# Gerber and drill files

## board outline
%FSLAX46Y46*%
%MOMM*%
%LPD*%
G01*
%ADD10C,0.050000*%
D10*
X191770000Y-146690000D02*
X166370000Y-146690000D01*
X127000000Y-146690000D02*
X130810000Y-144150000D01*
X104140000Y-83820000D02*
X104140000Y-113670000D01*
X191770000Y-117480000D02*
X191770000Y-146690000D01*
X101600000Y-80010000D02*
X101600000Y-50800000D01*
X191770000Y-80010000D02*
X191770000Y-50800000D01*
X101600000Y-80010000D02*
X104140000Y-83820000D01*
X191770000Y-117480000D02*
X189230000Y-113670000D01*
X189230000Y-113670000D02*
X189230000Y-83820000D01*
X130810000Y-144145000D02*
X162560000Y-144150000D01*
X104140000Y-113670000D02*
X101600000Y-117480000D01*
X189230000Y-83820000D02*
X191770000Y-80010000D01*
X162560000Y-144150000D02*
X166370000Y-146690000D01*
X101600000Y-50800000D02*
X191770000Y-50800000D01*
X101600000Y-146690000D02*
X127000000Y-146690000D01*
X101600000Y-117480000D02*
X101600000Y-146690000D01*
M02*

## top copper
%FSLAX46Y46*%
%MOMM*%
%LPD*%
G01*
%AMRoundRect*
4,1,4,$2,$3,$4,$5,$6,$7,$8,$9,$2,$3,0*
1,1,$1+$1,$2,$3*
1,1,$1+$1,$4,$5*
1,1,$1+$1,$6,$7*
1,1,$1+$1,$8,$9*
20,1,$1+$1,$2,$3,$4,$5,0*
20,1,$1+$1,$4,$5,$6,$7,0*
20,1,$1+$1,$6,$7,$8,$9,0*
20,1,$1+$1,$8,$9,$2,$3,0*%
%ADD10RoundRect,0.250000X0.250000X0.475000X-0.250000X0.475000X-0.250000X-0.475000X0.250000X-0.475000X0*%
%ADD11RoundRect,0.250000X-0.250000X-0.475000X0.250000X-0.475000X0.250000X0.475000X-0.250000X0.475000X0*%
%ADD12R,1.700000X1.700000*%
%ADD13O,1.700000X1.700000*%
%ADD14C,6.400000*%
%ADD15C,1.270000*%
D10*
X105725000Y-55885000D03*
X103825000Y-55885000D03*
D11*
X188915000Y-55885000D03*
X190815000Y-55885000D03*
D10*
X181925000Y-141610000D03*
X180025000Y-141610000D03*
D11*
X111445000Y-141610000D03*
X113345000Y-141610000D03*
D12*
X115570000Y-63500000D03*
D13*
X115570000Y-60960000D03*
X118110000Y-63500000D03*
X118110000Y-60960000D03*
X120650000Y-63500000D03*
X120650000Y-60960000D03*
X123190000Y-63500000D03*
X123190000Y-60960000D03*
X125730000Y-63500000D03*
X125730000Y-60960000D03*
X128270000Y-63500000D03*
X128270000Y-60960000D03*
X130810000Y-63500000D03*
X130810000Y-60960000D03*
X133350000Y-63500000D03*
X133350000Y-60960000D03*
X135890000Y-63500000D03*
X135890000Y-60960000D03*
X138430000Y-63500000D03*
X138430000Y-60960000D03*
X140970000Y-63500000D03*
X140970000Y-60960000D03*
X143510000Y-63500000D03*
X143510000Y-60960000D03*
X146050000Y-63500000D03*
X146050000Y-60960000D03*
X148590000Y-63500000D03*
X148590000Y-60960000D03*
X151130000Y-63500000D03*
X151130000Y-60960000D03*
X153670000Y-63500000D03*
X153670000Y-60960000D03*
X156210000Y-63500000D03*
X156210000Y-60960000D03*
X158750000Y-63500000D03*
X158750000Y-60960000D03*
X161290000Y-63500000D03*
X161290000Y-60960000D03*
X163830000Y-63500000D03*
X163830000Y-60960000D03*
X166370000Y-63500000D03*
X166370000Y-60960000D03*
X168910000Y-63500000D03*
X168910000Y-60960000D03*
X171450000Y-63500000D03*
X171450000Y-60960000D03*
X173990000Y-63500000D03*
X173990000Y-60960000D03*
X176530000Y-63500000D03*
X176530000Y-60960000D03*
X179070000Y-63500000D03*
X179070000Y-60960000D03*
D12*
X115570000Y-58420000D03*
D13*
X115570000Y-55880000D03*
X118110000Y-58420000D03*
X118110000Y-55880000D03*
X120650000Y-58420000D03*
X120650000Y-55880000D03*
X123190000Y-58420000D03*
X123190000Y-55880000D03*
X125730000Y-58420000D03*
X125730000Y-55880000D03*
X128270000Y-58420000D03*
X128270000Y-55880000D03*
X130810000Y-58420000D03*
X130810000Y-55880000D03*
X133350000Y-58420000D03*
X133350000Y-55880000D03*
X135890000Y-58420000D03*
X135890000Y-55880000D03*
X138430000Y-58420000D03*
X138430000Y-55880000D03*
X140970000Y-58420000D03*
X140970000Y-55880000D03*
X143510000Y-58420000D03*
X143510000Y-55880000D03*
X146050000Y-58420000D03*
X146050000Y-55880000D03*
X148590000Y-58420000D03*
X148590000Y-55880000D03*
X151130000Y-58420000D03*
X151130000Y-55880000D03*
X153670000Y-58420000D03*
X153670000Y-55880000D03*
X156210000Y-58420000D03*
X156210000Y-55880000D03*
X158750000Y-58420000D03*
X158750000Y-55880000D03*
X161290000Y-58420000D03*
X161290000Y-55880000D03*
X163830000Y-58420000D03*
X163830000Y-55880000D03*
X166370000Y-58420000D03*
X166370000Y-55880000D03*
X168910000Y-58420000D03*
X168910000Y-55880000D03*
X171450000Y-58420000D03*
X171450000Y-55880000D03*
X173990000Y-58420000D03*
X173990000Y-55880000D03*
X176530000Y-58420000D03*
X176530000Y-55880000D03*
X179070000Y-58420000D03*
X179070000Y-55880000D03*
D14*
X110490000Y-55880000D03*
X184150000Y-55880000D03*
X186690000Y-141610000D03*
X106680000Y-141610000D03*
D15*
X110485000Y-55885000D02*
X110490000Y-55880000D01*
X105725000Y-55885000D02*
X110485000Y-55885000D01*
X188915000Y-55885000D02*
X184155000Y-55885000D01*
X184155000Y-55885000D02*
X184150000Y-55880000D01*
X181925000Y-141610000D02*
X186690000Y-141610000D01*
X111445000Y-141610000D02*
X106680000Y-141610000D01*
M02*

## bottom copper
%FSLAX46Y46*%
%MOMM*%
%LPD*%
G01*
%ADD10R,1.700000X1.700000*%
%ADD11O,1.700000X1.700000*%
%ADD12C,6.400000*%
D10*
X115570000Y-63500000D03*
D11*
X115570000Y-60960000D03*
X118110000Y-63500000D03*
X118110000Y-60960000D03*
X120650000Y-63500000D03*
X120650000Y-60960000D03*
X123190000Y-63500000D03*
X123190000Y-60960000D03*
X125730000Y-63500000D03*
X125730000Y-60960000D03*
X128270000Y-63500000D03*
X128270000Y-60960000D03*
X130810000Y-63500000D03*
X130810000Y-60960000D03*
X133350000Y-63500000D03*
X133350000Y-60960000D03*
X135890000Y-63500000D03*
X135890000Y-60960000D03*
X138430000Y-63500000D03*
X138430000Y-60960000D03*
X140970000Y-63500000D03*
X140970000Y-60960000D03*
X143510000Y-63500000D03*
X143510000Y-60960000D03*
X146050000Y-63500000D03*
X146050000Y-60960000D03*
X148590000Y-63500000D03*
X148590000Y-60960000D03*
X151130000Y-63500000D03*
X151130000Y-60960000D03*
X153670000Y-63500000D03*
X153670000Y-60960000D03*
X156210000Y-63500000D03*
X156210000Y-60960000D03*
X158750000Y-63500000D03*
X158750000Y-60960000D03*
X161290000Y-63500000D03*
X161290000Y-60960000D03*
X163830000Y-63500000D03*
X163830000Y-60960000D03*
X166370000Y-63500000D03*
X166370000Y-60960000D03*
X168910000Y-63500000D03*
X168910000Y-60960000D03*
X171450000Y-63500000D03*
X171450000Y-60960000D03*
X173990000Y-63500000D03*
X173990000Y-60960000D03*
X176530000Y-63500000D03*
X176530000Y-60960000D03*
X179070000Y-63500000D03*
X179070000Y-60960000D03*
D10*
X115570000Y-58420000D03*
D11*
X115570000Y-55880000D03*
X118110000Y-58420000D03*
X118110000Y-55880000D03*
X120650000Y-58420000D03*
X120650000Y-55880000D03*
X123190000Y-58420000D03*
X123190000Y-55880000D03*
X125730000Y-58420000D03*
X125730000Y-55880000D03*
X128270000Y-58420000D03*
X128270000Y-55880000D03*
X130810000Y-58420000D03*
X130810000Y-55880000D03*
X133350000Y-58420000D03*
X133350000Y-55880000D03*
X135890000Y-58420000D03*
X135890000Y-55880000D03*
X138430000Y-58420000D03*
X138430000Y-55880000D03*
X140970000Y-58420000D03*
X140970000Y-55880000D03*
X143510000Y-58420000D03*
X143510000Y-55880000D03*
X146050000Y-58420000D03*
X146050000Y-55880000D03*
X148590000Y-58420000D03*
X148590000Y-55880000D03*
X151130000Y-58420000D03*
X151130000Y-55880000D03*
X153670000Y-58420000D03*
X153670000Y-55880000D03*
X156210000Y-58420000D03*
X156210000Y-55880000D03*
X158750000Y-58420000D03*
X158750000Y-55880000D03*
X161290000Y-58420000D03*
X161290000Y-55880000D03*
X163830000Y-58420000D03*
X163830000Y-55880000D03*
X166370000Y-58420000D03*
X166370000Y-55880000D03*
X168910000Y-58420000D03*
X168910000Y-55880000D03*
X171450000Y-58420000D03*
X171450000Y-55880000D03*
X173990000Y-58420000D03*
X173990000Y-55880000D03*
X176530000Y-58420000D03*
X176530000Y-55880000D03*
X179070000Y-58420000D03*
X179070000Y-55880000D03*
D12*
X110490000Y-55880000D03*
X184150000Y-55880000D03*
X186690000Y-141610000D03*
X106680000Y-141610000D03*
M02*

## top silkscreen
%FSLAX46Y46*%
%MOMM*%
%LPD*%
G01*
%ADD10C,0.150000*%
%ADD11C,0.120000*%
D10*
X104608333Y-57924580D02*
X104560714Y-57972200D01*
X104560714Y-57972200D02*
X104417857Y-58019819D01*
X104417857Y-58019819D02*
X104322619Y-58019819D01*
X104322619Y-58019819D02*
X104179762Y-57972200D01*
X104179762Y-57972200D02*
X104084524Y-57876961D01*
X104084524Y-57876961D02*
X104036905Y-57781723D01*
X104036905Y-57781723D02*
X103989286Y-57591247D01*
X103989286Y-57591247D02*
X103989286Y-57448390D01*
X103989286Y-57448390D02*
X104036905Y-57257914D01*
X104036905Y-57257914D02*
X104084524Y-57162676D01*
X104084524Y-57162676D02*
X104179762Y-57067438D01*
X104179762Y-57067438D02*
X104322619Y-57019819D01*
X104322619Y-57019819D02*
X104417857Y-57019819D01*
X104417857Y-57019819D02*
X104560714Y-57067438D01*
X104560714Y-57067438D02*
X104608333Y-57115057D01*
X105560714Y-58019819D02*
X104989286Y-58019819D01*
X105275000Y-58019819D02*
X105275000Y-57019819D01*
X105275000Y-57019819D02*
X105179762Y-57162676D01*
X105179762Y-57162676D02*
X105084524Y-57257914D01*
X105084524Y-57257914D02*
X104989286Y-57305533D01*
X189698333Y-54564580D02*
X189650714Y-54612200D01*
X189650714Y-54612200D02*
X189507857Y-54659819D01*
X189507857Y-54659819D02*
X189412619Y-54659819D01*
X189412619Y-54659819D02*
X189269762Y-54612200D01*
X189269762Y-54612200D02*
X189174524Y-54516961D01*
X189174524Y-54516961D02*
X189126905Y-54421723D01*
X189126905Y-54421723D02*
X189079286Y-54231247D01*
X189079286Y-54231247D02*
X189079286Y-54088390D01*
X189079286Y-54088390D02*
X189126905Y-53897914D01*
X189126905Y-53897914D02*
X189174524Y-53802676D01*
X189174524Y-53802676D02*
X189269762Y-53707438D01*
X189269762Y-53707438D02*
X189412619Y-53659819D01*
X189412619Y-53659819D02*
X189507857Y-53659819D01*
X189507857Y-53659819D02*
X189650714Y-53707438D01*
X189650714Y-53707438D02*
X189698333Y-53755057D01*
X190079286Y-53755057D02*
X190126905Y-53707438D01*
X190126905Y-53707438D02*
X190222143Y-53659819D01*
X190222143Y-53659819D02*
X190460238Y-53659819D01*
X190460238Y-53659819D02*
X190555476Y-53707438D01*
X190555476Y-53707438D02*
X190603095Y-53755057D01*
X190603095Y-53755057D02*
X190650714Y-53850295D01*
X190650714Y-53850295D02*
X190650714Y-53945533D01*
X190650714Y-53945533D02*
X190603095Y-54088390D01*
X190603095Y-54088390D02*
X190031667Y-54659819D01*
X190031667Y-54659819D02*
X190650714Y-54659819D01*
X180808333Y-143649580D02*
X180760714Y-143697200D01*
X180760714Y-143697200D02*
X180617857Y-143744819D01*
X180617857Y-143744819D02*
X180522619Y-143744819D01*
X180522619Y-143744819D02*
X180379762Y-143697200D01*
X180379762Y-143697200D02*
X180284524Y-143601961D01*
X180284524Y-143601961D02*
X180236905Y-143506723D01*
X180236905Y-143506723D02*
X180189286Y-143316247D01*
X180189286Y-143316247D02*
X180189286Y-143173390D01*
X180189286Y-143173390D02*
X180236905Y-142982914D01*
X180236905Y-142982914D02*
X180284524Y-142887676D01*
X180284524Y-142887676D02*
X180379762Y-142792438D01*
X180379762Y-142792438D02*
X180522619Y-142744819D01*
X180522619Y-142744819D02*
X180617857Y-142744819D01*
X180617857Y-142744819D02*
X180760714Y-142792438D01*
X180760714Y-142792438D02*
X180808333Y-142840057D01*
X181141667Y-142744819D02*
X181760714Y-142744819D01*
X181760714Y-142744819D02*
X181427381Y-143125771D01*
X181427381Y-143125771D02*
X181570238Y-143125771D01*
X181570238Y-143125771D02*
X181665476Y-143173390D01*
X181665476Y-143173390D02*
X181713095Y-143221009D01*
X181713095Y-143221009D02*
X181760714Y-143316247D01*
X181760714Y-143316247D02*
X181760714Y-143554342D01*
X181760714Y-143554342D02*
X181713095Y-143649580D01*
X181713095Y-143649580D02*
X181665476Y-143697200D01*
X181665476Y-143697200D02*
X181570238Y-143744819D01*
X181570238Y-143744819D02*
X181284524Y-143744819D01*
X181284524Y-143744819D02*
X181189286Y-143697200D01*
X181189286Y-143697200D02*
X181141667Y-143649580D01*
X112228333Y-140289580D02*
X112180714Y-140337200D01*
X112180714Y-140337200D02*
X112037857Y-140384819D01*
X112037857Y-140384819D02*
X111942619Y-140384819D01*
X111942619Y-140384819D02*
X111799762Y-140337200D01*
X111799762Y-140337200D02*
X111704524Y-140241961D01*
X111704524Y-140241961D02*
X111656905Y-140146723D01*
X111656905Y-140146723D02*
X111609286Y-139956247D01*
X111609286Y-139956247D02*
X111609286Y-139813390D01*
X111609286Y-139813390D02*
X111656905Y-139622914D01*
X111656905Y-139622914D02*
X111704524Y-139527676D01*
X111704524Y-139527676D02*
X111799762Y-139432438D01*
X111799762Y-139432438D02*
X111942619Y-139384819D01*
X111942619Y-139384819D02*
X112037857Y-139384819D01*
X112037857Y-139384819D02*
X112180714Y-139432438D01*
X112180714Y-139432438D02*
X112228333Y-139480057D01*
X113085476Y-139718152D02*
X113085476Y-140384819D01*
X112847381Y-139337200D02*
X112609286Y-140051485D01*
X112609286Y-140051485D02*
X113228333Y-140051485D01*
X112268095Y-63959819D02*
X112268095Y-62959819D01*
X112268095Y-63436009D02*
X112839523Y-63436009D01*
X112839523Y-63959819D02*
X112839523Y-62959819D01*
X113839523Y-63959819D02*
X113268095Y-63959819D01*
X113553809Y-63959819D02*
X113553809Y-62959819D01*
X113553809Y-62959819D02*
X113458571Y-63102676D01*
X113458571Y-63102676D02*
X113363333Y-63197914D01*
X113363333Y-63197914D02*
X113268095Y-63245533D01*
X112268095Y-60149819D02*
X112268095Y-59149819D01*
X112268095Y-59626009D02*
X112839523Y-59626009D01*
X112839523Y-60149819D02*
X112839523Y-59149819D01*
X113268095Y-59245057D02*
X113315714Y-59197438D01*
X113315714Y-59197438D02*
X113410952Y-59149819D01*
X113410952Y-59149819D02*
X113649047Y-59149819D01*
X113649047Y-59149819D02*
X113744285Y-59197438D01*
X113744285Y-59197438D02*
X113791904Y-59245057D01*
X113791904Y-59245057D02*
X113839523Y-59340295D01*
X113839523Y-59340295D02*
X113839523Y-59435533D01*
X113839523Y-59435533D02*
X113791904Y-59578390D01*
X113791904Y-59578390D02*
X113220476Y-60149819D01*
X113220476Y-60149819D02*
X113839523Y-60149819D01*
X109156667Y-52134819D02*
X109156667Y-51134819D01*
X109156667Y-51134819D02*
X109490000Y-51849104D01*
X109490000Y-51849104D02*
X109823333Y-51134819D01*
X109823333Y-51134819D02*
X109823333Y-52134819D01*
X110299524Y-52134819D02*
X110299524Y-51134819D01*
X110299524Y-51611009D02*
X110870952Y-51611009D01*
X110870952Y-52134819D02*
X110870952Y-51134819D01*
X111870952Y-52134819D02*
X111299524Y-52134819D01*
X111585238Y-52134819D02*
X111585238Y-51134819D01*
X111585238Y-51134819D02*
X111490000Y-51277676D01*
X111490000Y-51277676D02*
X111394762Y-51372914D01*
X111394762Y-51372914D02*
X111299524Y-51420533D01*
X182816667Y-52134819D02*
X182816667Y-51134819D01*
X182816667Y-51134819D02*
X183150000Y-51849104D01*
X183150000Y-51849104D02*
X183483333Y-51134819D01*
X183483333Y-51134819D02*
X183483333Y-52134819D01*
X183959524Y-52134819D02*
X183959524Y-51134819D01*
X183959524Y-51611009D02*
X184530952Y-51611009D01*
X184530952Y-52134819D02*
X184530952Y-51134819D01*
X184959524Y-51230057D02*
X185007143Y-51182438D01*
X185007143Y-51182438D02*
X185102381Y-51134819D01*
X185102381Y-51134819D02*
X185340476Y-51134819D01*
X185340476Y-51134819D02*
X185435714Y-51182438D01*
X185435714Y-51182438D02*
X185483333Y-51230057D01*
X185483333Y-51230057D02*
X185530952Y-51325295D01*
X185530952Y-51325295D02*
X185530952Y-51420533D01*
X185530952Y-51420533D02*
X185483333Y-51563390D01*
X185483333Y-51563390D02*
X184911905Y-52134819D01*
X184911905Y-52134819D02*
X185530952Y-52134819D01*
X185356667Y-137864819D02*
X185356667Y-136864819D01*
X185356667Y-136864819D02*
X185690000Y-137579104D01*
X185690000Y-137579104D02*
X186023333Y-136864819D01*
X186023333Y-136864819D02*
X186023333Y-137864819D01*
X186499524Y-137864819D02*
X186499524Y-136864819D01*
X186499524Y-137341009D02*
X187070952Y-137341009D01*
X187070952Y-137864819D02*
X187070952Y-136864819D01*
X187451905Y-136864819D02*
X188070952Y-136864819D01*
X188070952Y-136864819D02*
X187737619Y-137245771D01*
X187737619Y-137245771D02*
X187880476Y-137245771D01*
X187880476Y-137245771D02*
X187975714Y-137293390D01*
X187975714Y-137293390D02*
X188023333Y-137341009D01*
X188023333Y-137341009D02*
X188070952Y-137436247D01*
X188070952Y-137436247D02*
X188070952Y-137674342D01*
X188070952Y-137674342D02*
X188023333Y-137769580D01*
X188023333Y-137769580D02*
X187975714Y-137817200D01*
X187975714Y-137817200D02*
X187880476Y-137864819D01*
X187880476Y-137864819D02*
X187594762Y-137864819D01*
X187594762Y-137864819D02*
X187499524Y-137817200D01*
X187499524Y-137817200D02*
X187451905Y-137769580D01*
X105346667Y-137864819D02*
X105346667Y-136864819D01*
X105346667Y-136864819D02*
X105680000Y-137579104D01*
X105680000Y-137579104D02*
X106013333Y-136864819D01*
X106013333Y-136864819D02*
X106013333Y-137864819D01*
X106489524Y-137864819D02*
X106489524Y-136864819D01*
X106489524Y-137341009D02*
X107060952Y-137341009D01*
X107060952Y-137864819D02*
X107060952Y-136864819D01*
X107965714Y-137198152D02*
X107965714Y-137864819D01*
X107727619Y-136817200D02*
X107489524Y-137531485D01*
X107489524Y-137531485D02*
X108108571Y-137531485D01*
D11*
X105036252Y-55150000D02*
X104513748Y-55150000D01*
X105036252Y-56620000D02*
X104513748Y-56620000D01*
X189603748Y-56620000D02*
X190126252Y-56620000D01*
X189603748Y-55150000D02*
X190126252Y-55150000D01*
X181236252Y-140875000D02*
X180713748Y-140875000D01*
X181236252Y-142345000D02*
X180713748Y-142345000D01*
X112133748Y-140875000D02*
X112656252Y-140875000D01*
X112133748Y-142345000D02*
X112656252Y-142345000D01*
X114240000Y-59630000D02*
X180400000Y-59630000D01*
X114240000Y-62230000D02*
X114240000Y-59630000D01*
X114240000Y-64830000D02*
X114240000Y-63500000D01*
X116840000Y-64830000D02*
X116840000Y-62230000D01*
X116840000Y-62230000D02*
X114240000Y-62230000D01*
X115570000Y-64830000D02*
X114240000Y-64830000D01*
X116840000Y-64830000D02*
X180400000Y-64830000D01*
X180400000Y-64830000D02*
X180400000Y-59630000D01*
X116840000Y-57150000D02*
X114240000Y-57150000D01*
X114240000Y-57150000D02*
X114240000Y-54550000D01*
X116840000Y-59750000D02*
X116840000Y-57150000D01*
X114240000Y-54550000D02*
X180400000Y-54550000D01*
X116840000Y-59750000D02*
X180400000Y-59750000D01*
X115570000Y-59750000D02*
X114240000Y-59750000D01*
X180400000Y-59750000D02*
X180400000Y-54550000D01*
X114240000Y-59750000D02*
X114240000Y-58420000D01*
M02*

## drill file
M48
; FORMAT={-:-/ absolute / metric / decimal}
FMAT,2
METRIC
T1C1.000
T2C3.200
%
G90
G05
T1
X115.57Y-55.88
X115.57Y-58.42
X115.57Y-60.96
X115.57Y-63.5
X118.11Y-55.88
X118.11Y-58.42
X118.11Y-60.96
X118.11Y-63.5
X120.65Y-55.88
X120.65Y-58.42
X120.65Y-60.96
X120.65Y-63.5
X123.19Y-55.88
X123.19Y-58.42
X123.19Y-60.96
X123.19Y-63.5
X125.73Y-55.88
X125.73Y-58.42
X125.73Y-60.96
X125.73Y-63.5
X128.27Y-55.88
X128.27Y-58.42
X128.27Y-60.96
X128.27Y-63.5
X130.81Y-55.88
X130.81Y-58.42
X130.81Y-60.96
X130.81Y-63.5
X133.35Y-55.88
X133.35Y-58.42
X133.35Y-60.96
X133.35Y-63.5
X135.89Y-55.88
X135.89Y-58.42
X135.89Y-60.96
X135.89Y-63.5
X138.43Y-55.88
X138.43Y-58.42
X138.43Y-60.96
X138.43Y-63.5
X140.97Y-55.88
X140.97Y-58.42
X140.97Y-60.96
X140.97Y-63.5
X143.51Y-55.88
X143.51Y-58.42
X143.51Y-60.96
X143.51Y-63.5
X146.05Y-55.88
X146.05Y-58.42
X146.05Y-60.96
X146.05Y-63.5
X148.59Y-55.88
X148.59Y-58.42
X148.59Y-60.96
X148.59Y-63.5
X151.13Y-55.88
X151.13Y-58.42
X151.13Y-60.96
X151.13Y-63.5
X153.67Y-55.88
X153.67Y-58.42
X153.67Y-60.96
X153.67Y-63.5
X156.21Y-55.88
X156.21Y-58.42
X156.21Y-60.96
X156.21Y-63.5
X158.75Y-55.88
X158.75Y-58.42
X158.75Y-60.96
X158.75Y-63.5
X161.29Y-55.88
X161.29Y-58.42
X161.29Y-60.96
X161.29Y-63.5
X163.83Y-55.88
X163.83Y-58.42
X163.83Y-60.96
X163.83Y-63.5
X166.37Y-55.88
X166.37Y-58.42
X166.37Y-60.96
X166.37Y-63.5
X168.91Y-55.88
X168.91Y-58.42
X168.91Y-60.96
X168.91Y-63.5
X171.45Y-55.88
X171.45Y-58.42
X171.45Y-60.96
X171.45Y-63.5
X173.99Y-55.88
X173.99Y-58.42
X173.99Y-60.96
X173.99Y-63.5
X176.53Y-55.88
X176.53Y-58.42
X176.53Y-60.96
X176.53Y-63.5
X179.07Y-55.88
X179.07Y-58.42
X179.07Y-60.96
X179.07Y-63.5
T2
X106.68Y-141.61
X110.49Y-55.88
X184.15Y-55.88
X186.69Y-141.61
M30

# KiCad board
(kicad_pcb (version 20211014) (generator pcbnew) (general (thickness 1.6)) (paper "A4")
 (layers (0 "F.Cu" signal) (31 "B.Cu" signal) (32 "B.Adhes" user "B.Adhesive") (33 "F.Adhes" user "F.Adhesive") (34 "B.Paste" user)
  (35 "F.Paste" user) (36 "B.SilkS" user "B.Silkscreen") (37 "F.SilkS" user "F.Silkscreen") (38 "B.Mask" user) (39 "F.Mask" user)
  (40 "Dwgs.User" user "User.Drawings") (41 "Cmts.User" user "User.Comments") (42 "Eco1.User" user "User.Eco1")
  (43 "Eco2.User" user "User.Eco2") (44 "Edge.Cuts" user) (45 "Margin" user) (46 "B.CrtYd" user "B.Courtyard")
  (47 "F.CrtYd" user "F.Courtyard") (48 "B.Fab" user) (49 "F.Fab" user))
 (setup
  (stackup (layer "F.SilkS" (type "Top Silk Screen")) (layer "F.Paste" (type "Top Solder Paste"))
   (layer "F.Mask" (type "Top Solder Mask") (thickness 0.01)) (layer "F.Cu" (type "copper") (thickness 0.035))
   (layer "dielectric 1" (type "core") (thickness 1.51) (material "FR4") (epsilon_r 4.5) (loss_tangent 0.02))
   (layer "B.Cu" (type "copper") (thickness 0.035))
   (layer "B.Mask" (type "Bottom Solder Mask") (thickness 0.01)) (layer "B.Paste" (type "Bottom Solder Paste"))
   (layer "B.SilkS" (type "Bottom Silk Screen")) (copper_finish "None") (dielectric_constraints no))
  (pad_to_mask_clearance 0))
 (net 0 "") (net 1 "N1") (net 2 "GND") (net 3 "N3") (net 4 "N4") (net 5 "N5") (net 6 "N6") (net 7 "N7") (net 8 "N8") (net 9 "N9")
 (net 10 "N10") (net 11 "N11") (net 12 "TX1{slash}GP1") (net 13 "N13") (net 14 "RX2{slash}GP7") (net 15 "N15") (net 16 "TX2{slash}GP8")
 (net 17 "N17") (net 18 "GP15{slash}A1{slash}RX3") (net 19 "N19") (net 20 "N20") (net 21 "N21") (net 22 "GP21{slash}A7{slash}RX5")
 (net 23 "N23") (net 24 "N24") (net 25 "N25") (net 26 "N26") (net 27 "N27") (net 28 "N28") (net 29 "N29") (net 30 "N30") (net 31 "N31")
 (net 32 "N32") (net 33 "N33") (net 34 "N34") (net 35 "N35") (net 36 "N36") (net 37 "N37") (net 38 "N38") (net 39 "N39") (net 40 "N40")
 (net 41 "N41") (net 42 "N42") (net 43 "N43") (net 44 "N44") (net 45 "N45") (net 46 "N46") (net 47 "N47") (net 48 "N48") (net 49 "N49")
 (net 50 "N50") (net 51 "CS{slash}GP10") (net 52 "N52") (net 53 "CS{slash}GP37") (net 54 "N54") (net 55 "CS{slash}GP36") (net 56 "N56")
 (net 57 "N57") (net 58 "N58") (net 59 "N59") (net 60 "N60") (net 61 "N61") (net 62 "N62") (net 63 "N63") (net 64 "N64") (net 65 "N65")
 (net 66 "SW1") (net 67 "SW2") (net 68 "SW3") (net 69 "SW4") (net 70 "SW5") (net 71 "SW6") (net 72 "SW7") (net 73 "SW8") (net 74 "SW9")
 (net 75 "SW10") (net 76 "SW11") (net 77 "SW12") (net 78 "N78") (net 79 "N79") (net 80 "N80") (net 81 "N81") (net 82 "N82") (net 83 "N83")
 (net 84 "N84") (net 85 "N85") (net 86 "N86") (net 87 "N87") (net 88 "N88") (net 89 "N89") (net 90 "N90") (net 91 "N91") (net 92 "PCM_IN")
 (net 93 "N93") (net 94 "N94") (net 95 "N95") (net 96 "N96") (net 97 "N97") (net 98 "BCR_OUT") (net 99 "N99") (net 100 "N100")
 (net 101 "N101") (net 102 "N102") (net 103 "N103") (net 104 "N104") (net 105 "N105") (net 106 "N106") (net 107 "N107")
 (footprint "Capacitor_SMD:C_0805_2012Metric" (layer "F.Cu") (at 104.775 55.885 180)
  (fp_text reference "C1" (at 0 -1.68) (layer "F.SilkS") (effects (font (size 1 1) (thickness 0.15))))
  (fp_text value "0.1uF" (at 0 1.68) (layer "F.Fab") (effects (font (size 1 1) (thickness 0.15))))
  (fp_line (start -0.261252 0.735) (end 0.261252 0.735) (layer "F.SilkS") (width 0.12))
  (fp_line (start -0.261252 -0.735) (end 0.261252 -0.735) (layer "F.SilkS") (width 0.12))
  (pad "1" smd roundrect locked (at -0.95 0 180) (size 1 1.45) (layers "F.Cu" "F.Paste" "F.Mask") (roundrect_rratio 0.25) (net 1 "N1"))
  (pad "2" smd roundrect locked (at 0.95 0 180) (size 1 1.45) (layers "F.Cu" "F.Paste" "F.Mask") (roundrect_rratio 0.25) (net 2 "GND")))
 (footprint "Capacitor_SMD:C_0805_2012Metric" (layer "F.Cu") (at 189.865 55.885)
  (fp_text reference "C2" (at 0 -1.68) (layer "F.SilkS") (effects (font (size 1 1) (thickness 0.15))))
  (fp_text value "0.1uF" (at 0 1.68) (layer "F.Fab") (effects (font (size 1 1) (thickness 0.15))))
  (fp_line (start -0.261252 0.735) (end 0.261252 0.735) (layer "F.SilkS") (width 0.12))
  (fp_line (start -0.261252 -0.735) (end 0.261252 -0.735) (layer "F.SilkS") (width 0.12))
  (pad "1" smd roundrect locked (at -0.95 0) (size 1 1.45) (layers "F.Cu" "F.Paste" "F.Mask") (roundrect_rratio 0.25) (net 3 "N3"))
  (pad "2" smd roundrect locked (at 0.95 0) (size 1 1.45) (layers "F.Cu" "F.Paste" "F.Mask") (roundrect_rratio 0.25) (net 2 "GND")))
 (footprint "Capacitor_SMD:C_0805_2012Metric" (layer "F.Cu") (at 180.975 141.61 180)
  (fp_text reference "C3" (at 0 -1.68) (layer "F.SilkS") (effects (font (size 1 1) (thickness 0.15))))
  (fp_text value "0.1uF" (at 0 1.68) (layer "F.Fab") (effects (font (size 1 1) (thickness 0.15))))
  (fp_line (start -0.261252 0.735) (end 0.261252 0.735) (layer "F.SilkS") (width 0.12))
  (fp_line (start -0.261252 -0.735) (end 0.261252 -0.735) (layer "F.SilkS") (width 0.12))
  (pad "1" smd roundrect locked (at -0.95 0 180) (size 1 1.45) (layers "F.Cu" "F.Paste" "F.Mask") (roundrect_rratio 0.25) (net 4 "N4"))
  (pad "2" smd roundrect locked (at 0.95 0 180) (size 1 1.45) (layers "F.Cu" "F.Paste" "F.Mask") (roundrect_rratio 0.25) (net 2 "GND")))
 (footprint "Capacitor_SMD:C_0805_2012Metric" (layer "F.Cu") (at 112.395 141.61)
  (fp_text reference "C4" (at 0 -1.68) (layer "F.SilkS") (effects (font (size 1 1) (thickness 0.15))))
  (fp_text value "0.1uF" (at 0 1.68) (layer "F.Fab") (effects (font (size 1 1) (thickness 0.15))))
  (fp_line (start -0.261252 -0.735) (end 0.261252 -0.735) (layer "F.SilkS") (width 0.12))
  (fp_line (start -0.261252 0.735) (end 0.261252 0.735) (layer "F.SilkS") (width 0.12))
  (pad "1" smd roundrect locked (at -0.95 0) (size 1 1.45) (layers "F.Cu" "F.Paste" "F.Mask") (roundrect_rratio 0.25) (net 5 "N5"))
  (pad "2" smd roundrect locked (at 0.95 0) (size 1 1.45) (layers "F.Cu" "F.Paste" "F.Mask") (roundrect_rratio 0.25) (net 2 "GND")))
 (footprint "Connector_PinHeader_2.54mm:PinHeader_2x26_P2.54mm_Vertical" (layer "F.Cu") (at 115.57 63.5 90)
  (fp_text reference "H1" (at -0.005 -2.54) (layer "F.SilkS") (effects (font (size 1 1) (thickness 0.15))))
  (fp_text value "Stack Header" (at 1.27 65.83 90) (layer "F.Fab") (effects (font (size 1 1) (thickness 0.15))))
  (fp_line (start 3.87 -1.33) (end 3.87 64.83) (layer "F.SilkS") (width 0.12))
  (fp_line (start 1.27 -1.33) (end 3.87 -1.33) (layer "F.SilkS") (width 0.12))
  (fp_line (start -1.33 -1.33) (end 0 -1.33) (layer "F.SilkS") (width 0.12))
  (fp_line (start -1.33 1.27) (end 1.27 1.27) (layer "F.SilkS") (width 0.12))
  (fp_line (start 1.27 1.27) (end 1.27 -1.33) (layer "F.SilkS") (width 0.12))
  (fp_line (start -1.33 0) (end -1.33 -1.33) (layer "F.SilkS") (width 0.12))
  (fp_line (start -1.33 1.27) (end -1.33 64.83) (layer "F.SilkS") (width 0.12))
  (fp_line (start -1.33 64.83) (end 3.87 64.83) (layer "F.SilkS") (width 0.12))
  (pad "1" thru_hole rect locked (at 0 0 90) (size 1.7 1.7) (drill 1) (layers *.Cu *.Mask) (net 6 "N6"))
  (pad "2" thru_hole oval locked (at 2.54 0 90) (size 1.7 1.7) (drill 1) (layers *.Cu *.Mask) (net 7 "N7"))
  (pad "3" thru_hole oval locked (at 0 2.54 90) (size 1.7 1.7) (drill 1) (layers *.Cu *.Mask) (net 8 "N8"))
  (pad "4" thru_hole oval locked (at 2.54 2.54 90) (size 1.7 1.7) (drill 1) (layers *.Cu *.Mask) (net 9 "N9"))
  (pad "5" thru_hole oval locked (at 0 5.08 90) (size 1.7 1.7) (drill 1) (layers *.Cu *.Mask) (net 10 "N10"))
  (pad "6" thru_hole oval locked (at 2.54 5.08 90) (size 1.7 1.7) (drill 1) (layers *.Cu *.Mask) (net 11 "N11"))
  (pad "7" thru_hole oval locked (at 0 7.62 90) (size 1.7 1.7) (drill 1) (layers *.Cu *.Mask) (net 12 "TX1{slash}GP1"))
  (pad "8" thru_hole oval locked (at 2.54 7.62 90) (size 1.7 1.7) (drill 1) (layers *.Cu *.Mask) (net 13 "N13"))
  (pad "9" thru_hole oval locked (at 0 10.16 90) (size 1.7 1.7) (drill 1) (layers *.Cu *.Mask) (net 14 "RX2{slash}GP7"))
  (pad "10" thru_hole oval locked (at 2.54 10.16 90) (size 1.7 1.7) (drill 1) (layers *.Cu *.Mask) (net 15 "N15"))
  (pad "11" thru_hole oval locked (at 0 12.7 90) (size 1.7 1.7) (drill 1) (layers *.Cu *.Mask) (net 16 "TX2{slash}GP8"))
  (pad "12" thru_hole oval locked (at 2.54 12.7 90) (size 1.7 1.7) (drill 1) (layers *.Cu *.Mask) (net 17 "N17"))
  (pad "13" thru_hole oval locked (at 0 15.24 90) (size 1.7 1.7) (drill 1) (layers *.Cu *.Mask) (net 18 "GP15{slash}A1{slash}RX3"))
  (pad "14" thru_hole oval locked (at 2.54 15.24 90) (size 1.7 1.7) (drill 1) (layers *.Cu *.Mask) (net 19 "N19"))
  (pad "15" thru_hole oval locked (at 0 17.78 90) (size 1.7 1.7) (drill 1) (layers *.Cu *.Mask) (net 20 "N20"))
  (pad "16" thru_hole oval locked (at 2.54 17.78 90) (size 1.7 1.7) (drill 1) (layers *.Cu *.Mask) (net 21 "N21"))
  (pad "17" thru_hole oval locked (at 0 20.32 90) (size 1.7 1.7) (drill 1) (layers *.Cu *.Mask) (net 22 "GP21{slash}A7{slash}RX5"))
  (pad "18" thru_hole oval locked (at 2.54 20.32 90) (size 1.7 1.7) (drill 1) (layers *.Cu *.Mask) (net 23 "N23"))
  (pad "19" thru_hole oval locked (at 0 22.86 90) (size 1.7 1.7) (drill 1) (layers *.Cu *.Mask) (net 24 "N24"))
  (pad "20" thru_hole oval locked (at 2.54 22.86 90) (size 1.7 1.7) (drill 1) (layers *.Cu *.Mask) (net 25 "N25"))
  (pad "21" thru_hole oval locked (at 0 25.4 90) (size 1.7 1.7) (drill 1) (layers *.Cu *.Mask) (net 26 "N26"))
  (pad "22" thru_hole oval locked (at 2.54 25.4 90) (size 1.7 1.7) (drill 1) (layers *.Cu *.Mask) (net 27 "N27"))
  (pad "23" thru_hole oval locked (at 0 27.94 90) (size 1.7 1.7) (drill 1) (layers *.Cu *.Mask) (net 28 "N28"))
  (pad "24" thru_hole oval locked (at 2.54 27.94 90) (size 1.7 1.7) (drill 1) (layers *.Cu *.Mask) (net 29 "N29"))
  (pad "25" thru_hole oval locked (at 0 30.48 90) (size 1.7 1.7) (drill 1) (layers *.Cu *.Mask) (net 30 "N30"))
  (pad "26" thru_hole oval locked (at 2.54 30.48 90) (size 1.7 1.7) (drill 1) (layers *.Cu *.Mask) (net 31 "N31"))
  (pad "27" thru_hole oval locked (at 0 33.02 90) (size 1.7 1.7) (drill 1) (layers *.Cu *.Mask) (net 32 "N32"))
  (pad "28" thru_hole oval locked (at 2.54 33.02 90) (size 1.7 1.7) (drill 1) (layers *.Cu *.Mask) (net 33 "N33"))
  (pad "29" thru_hole oval locked (at 0 35.56 90) (size 1.7 1.7) (drill 1) (layers *.Cu *.Mask) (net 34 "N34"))
  (pad "30" thru_hole oval locked (at 2.54 35.56 90) (size 1.7 1.7) (drill 1) (layers *.Cu *.Mask) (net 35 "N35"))
  (pad "31" thru_hole oval locked (at 0 38.1 90) (size 1.7 1.7) (drill 1) (layers *.Cu *.Mask) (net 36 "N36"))
  (pad "32" thru_hole oval locked (at 2.54 38.1 90) (size 1.7 1.7) (drill 1) (layers *.Cu *.Mask) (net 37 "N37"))
  (pad "33" thru_hole oval locked (at 0 40.64 90) (size 1.7 1.7) (drill 1) (layers *.Cu *.Mask) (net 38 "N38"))
  (pad "34" thru_hole oval locked (at 2.54 40.64 90) (size 1.7 1.7) (drill 1) (layers *.Cu *.Mask) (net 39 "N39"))
  (pad "35" thru_hole oval locked (at 0 43.18 90) (size 1.7 1.7) (drill 1) (layers *.Cu *.Mask) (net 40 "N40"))
  (pad "36" thru_hole oval locked (at 2.54 43.18 90) (size 1.7 1.7) (drill 1) (layers *.Cu *.Mask) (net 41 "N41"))
  (pad "37" thru_hole oval locked (at 0 45.72 90) (size 1.7 1.7) (drill 1) (layers *.Cu *.Mask) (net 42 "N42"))
  (pad "38" thru_hole oval locked (at 2.54 45.72 90) (size 1.7 1.7) (drill 1) (layers *.Cu *.Mask) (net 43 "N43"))
  (pad "39" thru_hole oval locked (at 0 48.26 90) (size 1.7 1.7) (drill 1) (layers *.Cu *.Mask) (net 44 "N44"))
  (pad "40" thru_hole oval locked (at 2.54 48.26 90) (size 1.7 1.7) (drill 1) (layers *.Cu *.Mask) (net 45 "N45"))
  (pad "41" thru_hole oval locked (at 0 50.8 90) (size 1.7 1.7) (drill 1) (layers *.Cu *.Mask) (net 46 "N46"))
  (pad "42" thru_hole oval locked (at 2.54 50.8 90) (size 1.7 1.7) (drill 1) (layers *.Cu *.Mask) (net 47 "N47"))
  (pad "43" thru_hole oval locked (at 0 53.34 90) (size 1.7 1.7) (drill 1) (layers *.Cu *.Mask) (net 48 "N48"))
  (pad "44" thru_hole oval locked (at 2.54 53.34 90) (size 1.7 1.7) (drill 1) (layers *.Cu *.Mask) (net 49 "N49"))
  (pad "45" thru_hole oval locked (at 0 55.88 90) (size 1.7 1.7) (drill 1) (layers *.Cu *.Mask) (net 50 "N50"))
  (pad "46" thru_hole oval locked (at 2.54 55.88 90) (size 1.7 1.7) (drill 1) (layers *.Cu *.Mask) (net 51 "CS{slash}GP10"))
  (pad "47" thru_hole oval locked (at 0 58.42 90) (size 1.7 1.7) (drill 1) (layers *.Cu *.Mask) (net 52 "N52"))
  (pad "48" thru_hole oval locked (at 2.54 58.42 90) (size 1.7 1.7) (drill 1) (layers *.Cu *.Mask) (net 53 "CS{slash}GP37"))
  (pad "49" thru_hole oval locked (at 0 60.96 90) (size 1.7 1.7) (drill 1) (layers *.Cu *.Mask) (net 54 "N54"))
  (pad "50" thru_hole oval locked (at 2.54 60.96 90) (size 1.7 1.7) (drill 1) (layers *.Cu *.Mask) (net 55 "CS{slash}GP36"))
  (pad "51" thru_hole oval locked (at 0 63.5 90) (size 1.7 1.7) (drill 1) (layers *.Cu *.Mask) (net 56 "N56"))
  (pad "52" thru_hole oval locked (at 2.54 63.5 90) (size 1.7 1.7) (drill 1) (layers *.Cu *.Mask) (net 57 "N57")))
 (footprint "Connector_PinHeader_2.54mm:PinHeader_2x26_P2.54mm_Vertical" (layer "F.Cu") (at 115.57 58.42 90)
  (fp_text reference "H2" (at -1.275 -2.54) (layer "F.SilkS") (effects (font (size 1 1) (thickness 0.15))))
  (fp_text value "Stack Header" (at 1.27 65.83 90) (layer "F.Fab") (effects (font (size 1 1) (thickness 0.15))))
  (fp_line (start 1.27 1.27) (end 1.27 -1.33) (layer "F.SilkS") (width 0.12))
  (fp_line (start 1.27 -1.33) (end 3.87 -1.33) (layer "F.SilkS") (width 0.12))
  (fp_line (start -1.33 1.27) (end 1.27 1.27) (layer "F.SilkS") (width 0.12))
  (fp_line (start 3.87 -1.33) (end 3.87 64.83) (layer "F.SilkS") (width 0.12))
  (fp_line (start -1.33 1.27) (end -1.33 64.83) (layer "F.SilkS") (width 0.12))
  (fp_line (start -1.33 0) (end -1.33 -1.33) (layer "F.SilkS") (width 0.12))
  (fp_line (start -1.33 64.83) (end 3.87 64.83) (layer "F.SilkS") (width 0.12))
  (fp_line (start -1.33 -1.33) (end 0 -1.33) (layer "F.SilkS") (width 0.12))
  (pad "1" thru_hole rect locked (at 0 0 90) (size 1.7 1.7) (drill 1) (layers *.Cu *.Mask) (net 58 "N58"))
  (pad "2" thru_hole oval locked (at 2.54 0 90) (size 1.7 1.7) (drill 1) (layers *.Cu *.Mask) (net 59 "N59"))
  (pad "3" thru_hole oval locked (at 0 2.54 90) (size 1.7 1.7) (drill 1) (layers *.Cu *.Mask) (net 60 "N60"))
  (pad "4" thru_hole oval locked (at 2.54 2.54 90) (size 1.7 1.7) (drill 1) (layers *.Cu *.Mask) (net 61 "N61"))
  (pad "5" thru_hole oval locked (at 0 5.08 90) (size 1.7 1.7) (drill 1) (layers *.Cu *.Mask) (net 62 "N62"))
  (pad "6" thru_hole oval locked (at 2.54 5.08 90) (size 1.7 1.7) (drill 1) (layers *.Cu *.Mask) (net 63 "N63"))
  (pad "7" thru_hole oval locked (at 0 7.62 90) (size 1.7 1.7) (drill 1) (layers *.Cu *.Mask) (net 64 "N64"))
  (pad "8" thru_hole oval locked (at 2.54 7.62 90) (size 1.7 1.7) (drill 1) (layers *.Cu *.Mask) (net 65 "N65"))
  (pad "9" thru_hole oval locked (at 0 10.16 90) (size 1.7 1.7) (drill 1) (layers *.Cu *.Mask) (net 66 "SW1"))
  (pad "10" thru_hole oval locked (at 2.54 10.16 90) (size 1.7 1.7) (drill 1) (layers *.Cu *.Mask) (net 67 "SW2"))
  (pad "11" thru_hole oval locked (at 0 12.7 90) (size 1.7 1.7) (drill 1) (layers *.Cu *.Mask) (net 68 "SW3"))
  (pad "12" thru_hole oval locked (at 2.54 12.7 90) (size 1.7 1.7) (drill 1) (layers *.Cu *.Mask) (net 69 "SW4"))
  (pad "13" thru_hole oval locked (at 0 15.24 90) (size 1.7 1.7) (drill 1) (layers *.Cu *.Mask) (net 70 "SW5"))
  (pad "14" thru_hole oval locked (at 2.54 15.24 90) (size 1.7 1.7) (drill 1) (layers *.Cu *.Mask) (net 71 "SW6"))
  (pad "15" thru_hole oval locked (at 0 17.78 90) (size 1.7 1.7) (drill 1) (layers *.Cu *.Mask) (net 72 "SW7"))
  (pad "16" thru_hole oval locked (at 2.54 17.78 90) (size 1.7 1.7) (drill 1) (layers *.Cu *.Mask) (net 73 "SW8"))
  (pad "17" thru_hole oval locked (at 0 20.32 90) (size 1.7 1.7) (drill 1) (layers *.Cu *.Mask) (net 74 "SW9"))
  (pad "18" thru_hole oval locked (at 2.54 20.32 90) (size 1.7 1.7) (drill 1) (layers *.Cu *.Mask) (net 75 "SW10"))
  (pad "19" thru_hole oval locked (at 0 22.86 90) (size 1.7 1.7) (drill 1) (layers *.Cu *.Mask) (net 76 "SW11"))
  (pad "20" thru_hole oval locked (at 2.54 22.86 90) (size 1.7 1.7) (drill 1) (layers *.Cu *.Mask) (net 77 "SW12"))
  (pad "21" thru_hole oval locked (at 0 25.4 90) (size 1.7 1.7) (drill 1) (layers *.Cu *.Mask) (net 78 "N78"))
  (pad "22" thru_hole oval locked (at 2.54 25.4 90) (size 1.7 1.7) (drill 1) (layers *.Cu *.Mask) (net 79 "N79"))
  (pad "23" thru_hole oval locked (at 0 27.94 90) (size 1.7 1.7) (drill 1) (layers *.Cu *.Mask) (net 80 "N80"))
  (pad "24" thru_hole oval locked (at 2.54 27.94 90) (size 1.7 1.7) (drill 1) (layers *.Cu *.Mask) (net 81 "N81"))
  (pad "25" thru_hole oval locked (at 0 30.48 90) (size 1.7 1.7) (drill 1) (layers *.Cu *.Mask) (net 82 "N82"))
  (pad "26" thru_hole oval locked (at 2.54 30.48 90) (size 1.7 1.7) (drill 1) (layers *.Cu *.Mask) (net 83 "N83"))
  (pad "27" thru_hole oval locked (at 0 33.02 90) (size 1.7 1.7) (drill 1) (layers *.Cu *.Mask) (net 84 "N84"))
  (pad "28" thru_hole oval locked (at 2.54 33.02 90) (size 1.7 1.7) (drill 1) (layers *.Cu *.Mask) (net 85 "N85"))
  (pad "29" thru_hole oval locked (at 0 35.56 90) (size 1.7 1.7) (drill 1) (layers *.Cu *.Mask) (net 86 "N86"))
  (pad "30" thru_hole oval locked (at 2.54 35.56 90) (size 1.7 1.7) (drill 1) (layers *.Cu *.Mask) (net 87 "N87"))
  (pad "31" thru_hole oval locked (at 0 38.1 90) (size 1.7 1.7) (drill 1) (layers *.Cu *.Mask) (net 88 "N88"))
  (pad "32" thru_hole oval locked (at 2.54 38.1 90) (size 1.7 1.7) (drill 1) (layers *.Cu *.Mask) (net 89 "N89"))
  (pad "33" thru_hole oval locked (at 0 40.64 90) (size 1.7 1.7) (drill 1) (layers *.Cu *.Mask) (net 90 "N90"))
  (pad "34" thru_hole oval locked (at 2.54 40.64 90) (size 1.7 1.7) (drill 1) (layers *.Cu *.Mask) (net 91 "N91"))
  (pad "35" thru_hole oval locked (at 0 43.18 90) (size 1.7 1.7) (drill 1) (layers *.Cu *.Mask) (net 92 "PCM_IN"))
  (pad "36" thru_hole oval locked (at 2.54 43.18 90) (size 1.7 1.7) (drill 1) (layers *.Cu *.Mask) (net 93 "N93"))
  (pad "37" thru_hole oval locked (at 0 45.72 90) (size 1.7 1.7) (drill 1) (layers *.Cu *.Mask) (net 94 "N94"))
  (pad "38" thru_hole oval locked (at 2.54 45.72 90) (size 1.7 1.7) (drill 1) (layers *.Cu *.Mask) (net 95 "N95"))
  (pad "39" thru_hole oval locked (at 0 48.26 90) (size 1.7 1.7) (drill 1) (layers *.Cu *.Mask) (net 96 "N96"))
  (pad "40" thru_hole oval locked (at 2.54 48.26 90) (size 1.7 1.7) (drill 1) (layers *.Cu *.Mask) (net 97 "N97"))
  (pad "41" thru_hole oval locked (at 0 50.8 90) (size 1.7 1.7) (drill 1) (layers *.Cu *.Mask) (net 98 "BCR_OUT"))
  (pad "42" thru_hole oval locked (at 2.54 50.8 90) (size 1.7 1.7) (drill 1) (layers *.Cu *.Mask) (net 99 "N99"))
  (pad "43" thru_hole oval locked (at 0 53.34 90) (size 1.7 1.7) (drill 1) (layers *.Cu *.Mask) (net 98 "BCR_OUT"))
  (pad "44" thru_hole oval locked (at 2.54 53.34 90) (size 1.7 1.7) (drill 1) (layers *.Cu *.Mask) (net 98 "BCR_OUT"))
  (pad "45" thru_hole oval locked (at 0 55.88 90) (size 1.7 1.7) (drill 1) (layers *.Cu *.Mask) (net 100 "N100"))
  (pad "46" thru_hole oval locked (at 2.54 55.88 90) (size 1.7 1.7) (drill 1) (layers *.Cu *.Mask) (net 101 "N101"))
  (pad "47" thru_hole oval locked (at 0 58.42 90) (size 1.7 1.7) (drill 1) (layers *.Cu *.Mask) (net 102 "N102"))
  (pad "48" thru_hole oval locked (at 2.54 58.42 90) (size 1.7 1.7) (drill 1) (layers *.Cu *.Mask) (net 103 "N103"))
  (pad "49" thru_hole oval locked (at 0 60.96 90) (size 1.7 1.7) (drill 1) (layers *.Cu *.Mask) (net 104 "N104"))
  (pad "50" thru_hole oval locked (at 2.54 60.96 90) (size 1.7 1.7) (drill 1) (layers *.Cu *.Mask) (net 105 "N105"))
  (pad "51" thru_hole oval locked (at 0 63.5 90) (size 1.7 1.7) (drill 1) (layers *.Cu *.Mask) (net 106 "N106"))
  (pad "52" thru_hole oval locked (at 2.54 63.5 90) (size 1.7 1.7) (drill 1) (layers *.Cu *.Mask) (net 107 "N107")))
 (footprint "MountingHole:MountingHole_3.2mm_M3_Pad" (layer "F.Cu") (at 110.49 55.88)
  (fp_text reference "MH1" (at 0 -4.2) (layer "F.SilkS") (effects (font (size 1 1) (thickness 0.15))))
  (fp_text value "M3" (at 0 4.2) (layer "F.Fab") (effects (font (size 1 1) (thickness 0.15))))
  (pad "1" thru_hole circle locked (at 0 0) (size 6.4 6.4) (drill 3.2) (layers *.Cu *.Mask) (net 1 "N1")))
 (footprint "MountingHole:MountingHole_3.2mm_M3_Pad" (layer "F.Cu") (at 184.15 55.88)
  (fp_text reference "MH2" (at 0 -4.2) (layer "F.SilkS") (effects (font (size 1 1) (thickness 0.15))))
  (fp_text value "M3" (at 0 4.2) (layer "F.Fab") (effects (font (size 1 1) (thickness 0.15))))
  (pad "1" thru_hole circle locked (at 0 0) (size 6.4 6.4) (drill 3.2) (layers *.Cu *.Mask) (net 3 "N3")))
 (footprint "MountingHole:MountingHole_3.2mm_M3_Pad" (layer "F.Cu") (at 186.69 141.61)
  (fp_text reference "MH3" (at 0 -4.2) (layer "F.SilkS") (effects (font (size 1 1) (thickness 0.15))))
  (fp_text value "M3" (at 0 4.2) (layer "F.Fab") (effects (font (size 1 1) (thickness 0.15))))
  (pad "1" thru_hole circle locked (at 0 0) (size 6.4 6.4) (drill 3.2) (layers *.Cu *.Mask) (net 4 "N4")))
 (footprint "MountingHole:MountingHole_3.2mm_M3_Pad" (layer "F.Cu") (at 106.68 141.61)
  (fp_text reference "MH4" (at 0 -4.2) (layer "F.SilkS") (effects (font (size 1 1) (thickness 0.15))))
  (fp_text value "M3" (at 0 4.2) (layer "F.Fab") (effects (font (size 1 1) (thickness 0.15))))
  (pad "1" thru_hole circle locked (at 0 0) (size 6.4 6.4) (drill 3.2) (layers *.Cu *.Mask) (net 5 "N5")))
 (gr_line (start 191.77 146.69) (end 166.37 146.69) (layer "Edge.Cuts") (width 0.05))
 (gr_line (start 127 146.69) (end 130.81 144.15) (layer "Edge.Cuts") (width 0.05))
 (gr_line (start 104.14 83.82) (end 104.14 113.67) (layer "Edge.Cuts") (width 0.05))
 (gr_line (start 191.77 117.48) (end 191.77 146.69) (layer "Edge.Cuts") (width 0.05))
 (gr_line (start 101.6 80.01) (end 101.6 50.8) (layer "Edge.Cuts") (width 0.05))
 (gr_line (start 191.77 80.01) (end 191.77 50.8) (layer "Edge.Cuts") (width 0.05))
 (gr_line (start 101.6 80.01) (end 104.14 83.82) (layer "Edge.Cuts") (width 0.05))
 (gr_line (start 191.77 117.48) (end 189.23 113.67) (layer "Edge.Cuts") (width 0.05))
 (gr_line (start 189.23 113.67) (end 189.23 83.82) (layer "Edge.Cuts") (width 0.05))
 (gr_line (start 130.81 144.145) (end 162.56 144.15) (layer "Edge.Cuts") (width 0.05))
 (gr_line (start 104.14 113.67) (end 101.6 117.48) (layer "Edge.Cuts") (width 0.05))
 (gr_line (start 189.23 83.82) (end 191.77 80.01) (layer "Edge.Cuts") (width 0.05))
 (gr_line (start 162.56 144.15) (end 166.37 146.69) (layer "Edge.Cuts") (width 0.05))
 (gr_line (start 101.6 50.8) (end 191.77 50.8) (layer "Edge.Cuts") (width 0.05))
 (gr_line (start 101.6 146.69) (end 127 146.69) (layer "Edge.Cuts") (width 0.05))
 (gr_line (start 101.6 117.48) (end 101.6 146.69) (layer "Edge.Cuts") (width 0.05))
 (segment (start 110.485 55.885) (end 110.49 55.88) (width 1.27) (layer "F.Cu") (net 1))
 (segment (start 105.725 55.885) (end 110.485 55.885) (width 1.27) (layer "F.Cu") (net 1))
 (segment (start 188.915 55.885) (end 184.155 55.885) (width 1.27) (layer "F.Cu") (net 3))
 (segment (start 184.155 55.885) (end 184.15 55.88) (width 1.27) (layer "F.Cu") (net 3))
 (segment (start 181.925 141.61) (end 186.69 141.61) (width 1.27) (layer "F.Cu") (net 4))
 (segment (start 111.445 141.61) (end 106.68 141.61) (width 1.27) (layer "F.Cu") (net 5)))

